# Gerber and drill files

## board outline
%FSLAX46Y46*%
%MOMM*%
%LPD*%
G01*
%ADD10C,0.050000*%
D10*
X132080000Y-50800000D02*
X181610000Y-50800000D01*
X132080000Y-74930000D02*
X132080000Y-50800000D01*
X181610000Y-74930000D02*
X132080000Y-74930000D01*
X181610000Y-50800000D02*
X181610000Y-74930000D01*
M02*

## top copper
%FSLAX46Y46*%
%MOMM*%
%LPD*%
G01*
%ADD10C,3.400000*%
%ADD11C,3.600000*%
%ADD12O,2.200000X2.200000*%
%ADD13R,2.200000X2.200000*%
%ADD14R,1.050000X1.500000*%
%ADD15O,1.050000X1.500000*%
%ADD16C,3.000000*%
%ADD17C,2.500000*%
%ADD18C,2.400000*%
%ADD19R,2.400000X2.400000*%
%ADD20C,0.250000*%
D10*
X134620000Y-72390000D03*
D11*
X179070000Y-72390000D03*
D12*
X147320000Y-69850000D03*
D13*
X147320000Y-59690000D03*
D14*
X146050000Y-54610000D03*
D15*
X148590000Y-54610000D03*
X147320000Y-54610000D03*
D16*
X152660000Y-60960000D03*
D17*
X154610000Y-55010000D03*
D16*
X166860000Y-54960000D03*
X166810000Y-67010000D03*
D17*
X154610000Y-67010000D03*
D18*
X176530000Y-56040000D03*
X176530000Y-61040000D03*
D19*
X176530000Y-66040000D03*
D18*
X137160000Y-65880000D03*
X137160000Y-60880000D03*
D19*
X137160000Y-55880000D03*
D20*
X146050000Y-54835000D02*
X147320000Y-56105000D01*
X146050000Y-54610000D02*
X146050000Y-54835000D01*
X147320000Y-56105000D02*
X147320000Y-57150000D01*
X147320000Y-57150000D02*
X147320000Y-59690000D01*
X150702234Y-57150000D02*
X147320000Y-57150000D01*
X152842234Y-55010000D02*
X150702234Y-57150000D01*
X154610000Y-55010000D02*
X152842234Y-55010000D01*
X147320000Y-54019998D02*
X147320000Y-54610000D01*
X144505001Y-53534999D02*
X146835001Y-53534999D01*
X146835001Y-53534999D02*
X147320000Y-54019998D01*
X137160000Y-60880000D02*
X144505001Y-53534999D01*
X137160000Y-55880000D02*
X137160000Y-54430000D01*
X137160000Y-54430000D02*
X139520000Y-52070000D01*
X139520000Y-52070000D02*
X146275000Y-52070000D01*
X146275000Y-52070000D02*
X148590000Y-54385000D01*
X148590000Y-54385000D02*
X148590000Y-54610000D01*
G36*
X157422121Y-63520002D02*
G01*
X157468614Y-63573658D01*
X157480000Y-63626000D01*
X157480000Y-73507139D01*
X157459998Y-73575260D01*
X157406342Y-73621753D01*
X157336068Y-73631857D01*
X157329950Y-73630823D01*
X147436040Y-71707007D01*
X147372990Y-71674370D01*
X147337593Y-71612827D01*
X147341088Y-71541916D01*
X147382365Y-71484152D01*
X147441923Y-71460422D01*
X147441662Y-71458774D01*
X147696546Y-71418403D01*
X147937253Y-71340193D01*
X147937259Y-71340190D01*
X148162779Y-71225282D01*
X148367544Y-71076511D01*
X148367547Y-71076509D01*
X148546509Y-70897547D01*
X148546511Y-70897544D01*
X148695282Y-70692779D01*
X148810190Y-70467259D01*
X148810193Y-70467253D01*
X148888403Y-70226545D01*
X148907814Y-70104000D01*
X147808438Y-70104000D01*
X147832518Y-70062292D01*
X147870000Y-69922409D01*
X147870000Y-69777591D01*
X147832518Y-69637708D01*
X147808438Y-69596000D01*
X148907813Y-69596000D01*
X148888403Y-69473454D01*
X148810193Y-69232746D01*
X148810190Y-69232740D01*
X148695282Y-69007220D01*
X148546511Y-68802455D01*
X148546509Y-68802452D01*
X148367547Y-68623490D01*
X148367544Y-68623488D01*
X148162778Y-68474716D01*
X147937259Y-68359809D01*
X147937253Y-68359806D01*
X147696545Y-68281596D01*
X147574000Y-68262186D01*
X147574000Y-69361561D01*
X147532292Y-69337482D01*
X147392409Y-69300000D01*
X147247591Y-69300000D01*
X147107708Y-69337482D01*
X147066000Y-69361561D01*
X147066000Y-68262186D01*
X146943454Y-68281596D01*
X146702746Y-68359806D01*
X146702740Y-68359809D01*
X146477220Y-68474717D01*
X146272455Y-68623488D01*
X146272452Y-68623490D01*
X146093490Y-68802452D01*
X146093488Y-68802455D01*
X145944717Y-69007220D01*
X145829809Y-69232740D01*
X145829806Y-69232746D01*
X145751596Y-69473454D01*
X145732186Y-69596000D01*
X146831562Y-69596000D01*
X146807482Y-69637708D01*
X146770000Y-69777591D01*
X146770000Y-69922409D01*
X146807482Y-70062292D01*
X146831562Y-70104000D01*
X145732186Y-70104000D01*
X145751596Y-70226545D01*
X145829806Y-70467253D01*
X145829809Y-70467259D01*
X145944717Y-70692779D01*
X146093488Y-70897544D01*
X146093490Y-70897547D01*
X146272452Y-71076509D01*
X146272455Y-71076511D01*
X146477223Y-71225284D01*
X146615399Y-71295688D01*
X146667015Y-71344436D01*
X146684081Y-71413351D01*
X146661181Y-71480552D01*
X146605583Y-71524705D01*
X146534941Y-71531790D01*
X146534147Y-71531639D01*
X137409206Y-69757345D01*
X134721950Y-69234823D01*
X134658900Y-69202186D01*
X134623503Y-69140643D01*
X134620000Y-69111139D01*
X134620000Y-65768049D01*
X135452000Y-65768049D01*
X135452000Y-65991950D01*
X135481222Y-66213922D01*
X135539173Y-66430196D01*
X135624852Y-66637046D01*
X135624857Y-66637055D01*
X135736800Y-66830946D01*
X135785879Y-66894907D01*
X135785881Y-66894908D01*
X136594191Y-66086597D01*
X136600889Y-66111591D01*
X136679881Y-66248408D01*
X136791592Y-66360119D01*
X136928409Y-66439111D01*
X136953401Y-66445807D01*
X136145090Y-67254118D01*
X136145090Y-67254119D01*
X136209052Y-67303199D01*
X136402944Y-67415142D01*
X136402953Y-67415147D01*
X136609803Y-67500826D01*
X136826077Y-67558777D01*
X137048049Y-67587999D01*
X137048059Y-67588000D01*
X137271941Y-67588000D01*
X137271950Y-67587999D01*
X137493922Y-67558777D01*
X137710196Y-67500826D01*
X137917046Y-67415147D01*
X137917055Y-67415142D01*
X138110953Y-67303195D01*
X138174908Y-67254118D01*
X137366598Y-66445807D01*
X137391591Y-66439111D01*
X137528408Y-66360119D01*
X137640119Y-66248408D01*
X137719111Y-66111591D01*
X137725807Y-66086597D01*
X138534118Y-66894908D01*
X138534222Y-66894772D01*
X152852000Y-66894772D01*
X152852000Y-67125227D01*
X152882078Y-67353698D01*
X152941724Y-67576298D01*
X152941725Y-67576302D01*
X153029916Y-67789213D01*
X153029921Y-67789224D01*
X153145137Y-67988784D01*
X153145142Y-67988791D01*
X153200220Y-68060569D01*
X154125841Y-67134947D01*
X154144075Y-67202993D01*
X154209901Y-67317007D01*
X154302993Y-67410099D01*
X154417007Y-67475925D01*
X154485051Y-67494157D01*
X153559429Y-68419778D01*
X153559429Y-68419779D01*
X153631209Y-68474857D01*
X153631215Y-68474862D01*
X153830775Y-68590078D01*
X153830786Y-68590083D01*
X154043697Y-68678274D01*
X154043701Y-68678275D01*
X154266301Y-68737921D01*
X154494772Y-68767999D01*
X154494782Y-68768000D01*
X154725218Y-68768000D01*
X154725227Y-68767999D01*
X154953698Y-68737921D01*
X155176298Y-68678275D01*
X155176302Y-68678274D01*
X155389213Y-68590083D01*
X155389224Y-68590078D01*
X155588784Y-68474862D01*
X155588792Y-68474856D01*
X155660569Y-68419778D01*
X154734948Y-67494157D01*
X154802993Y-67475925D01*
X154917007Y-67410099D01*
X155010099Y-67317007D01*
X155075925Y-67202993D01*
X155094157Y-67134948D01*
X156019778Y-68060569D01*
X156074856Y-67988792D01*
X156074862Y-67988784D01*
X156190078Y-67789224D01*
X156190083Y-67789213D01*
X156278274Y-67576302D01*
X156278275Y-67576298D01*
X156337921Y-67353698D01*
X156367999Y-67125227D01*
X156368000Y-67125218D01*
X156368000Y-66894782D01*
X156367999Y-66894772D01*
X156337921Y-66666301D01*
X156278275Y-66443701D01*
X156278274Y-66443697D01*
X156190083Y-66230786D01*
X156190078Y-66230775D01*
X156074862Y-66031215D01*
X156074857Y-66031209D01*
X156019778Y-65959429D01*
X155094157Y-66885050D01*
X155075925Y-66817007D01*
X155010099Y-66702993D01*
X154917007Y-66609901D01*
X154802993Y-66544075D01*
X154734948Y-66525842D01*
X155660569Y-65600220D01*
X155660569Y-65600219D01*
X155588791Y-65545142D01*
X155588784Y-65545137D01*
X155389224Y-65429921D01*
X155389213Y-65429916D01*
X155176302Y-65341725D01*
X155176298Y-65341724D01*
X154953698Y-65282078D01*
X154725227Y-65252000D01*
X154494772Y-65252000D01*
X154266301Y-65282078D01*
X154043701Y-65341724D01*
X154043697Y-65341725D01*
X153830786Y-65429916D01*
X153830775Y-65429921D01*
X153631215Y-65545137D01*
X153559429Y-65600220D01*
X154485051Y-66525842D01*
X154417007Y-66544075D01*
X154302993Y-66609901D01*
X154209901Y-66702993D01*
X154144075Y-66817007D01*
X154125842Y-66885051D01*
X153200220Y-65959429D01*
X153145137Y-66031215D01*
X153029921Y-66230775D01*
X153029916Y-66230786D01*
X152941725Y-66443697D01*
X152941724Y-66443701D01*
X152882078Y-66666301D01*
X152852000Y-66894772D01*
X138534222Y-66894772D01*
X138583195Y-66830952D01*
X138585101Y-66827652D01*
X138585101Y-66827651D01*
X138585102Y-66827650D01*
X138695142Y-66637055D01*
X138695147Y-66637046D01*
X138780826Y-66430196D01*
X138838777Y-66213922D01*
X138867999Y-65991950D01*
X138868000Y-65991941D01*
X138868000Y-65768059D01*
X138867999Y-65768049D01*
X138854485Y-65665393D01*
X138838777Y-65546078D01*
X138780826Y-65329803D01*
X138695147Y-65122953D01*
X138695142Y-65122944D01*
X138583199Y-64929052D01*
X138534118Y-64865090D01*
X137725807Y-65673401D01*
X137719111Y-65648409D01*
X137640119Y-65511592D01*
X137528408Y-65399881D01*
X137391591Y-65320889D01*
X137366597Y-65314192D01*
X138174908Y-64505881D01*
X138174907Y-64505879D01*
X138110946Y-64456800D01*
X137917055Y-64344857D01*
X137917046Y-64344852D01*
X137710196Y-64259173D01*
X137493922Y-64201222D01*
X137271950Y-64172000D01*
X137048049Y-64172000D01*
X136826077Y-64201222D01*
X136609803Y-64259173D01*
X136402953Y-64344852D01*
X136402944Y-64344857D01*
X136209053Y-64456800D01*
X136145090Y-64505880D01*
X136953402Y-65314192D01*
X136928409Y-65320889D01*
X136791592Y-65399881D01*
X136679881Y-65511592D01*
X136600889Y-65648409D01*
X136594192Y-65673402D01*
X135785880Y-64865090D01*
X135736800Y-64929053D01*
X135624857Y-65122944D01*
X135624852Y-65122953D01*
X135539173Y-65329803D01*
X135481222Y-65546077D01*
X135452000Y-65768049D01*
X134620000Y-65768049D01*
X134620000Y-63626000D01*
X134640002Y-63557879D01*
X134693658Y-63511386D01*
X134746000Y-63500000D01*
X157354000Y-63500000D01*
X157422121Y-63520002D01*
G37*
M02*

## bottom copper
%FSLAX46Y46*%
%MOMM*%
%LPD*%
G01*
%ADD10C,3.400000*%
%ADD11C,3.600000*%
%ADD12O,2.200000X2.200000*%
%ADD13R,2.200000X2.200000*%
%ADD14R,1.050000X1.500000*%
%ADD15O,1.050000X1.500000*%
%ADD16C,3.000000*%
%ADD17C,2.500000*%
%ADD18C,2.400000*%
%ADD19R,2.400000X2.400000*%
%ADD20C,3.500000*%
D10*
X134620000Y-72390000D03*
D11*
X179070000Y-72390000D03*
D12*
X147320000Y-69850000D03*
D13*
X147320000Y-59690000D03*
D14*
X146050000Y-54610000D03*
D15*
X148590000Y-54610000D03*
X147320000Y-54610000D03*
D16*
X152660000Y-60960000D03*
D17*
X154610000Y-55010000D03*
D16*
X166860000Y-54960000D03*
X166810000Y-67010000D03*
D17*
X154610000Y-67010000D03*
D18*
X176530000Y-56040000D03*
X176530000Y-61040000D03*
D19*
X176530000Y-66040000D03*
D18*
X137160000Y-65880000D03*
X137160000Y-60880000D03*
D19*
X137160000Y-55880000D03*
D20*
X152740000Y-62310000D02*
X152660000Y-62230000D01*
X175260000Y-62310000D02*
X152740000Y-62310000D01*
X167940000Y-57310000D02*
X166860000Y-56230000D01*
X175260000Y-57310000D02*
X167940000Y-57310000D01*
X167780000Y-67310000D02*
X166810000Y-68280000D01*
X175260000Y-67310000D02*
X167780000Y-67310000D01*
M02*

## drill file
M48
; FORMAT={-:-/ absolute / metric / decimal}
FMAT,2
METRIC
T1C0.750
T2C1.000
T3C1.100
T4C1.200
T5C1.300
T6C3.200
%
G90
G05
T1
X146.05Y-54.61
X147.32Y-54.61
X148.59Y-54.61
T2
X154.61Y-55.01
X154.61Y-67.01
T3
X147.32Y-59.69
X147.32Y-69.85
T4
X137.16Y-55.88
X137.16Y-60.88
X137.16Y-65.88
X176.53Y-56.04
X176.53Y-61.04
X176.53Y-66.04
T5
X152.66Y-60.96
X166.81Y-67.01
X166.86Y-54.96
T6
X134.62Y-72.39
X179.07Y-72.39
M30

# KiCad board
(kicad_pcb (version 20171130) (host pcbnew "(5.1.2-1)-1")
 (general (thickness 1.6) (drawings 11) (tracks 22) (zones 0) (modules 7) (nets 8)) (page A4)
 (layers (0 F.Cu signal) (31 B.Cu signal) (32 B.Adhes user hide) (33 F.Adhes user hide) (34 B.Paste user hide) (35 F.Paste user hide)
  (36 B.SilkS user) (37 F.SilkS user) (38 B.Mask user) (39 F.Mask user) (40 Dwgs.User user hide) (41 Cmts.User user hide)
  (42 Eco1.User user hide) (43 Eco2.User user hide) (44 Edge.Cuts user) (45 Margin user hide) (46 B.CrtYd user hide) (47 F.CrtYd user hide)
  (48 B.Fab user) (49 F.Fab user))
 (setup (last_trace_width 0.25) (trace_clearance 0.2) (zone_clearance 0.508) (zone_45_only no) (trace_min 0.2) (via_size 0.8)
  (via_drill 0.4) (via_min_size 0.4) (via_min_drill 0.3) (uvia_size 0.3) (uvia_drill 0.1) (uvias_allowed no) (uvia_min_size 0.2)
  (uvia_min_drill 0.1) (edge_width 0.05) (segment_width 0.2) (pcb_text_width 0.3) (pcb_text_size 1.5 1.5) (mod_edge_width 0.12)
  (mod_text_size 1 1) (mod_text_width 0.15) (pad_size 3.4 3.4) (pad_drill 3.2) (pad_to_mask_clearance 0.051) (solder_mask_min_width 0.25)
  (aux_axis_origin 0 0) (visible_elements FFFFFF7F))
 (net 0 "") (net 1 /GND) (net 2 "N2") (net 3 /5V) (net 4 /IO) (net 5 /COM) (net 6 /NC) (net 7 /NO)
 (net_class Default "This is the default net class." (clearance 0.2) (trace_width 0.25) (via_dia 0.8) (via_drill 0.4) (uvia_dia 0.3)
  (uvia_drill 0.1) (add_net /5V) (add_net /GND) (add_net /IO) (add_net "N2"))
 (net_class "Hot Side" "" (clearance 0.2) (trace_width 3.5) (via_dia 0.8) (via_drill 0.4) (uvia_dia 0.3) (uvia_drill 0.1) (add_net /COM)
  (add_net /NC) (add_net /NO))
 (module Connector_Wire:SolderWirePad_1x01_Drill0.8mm (layer F.Cu) (at 134.62 72.39)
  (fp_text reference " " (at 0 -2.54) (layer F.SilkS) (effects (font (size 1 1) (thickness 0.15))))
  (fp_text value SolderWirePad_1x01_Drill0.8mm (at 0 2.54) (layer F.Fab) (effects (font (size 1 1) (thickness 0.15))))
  (pad 1 thru_hole circle (at 0 0) (size 3.4 3.4) (drill 3.2) (layers *.Cu *.Mask)))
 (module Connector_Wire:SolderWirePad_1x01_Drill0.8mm (layer F.Cu) (at 179.07 72.39)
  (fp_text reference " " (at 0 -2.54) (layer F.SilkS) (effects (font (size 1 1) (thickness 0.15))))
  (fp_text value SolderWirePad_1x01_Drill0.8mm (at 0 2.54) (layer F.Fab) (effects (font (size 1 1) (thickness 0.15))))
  (pad 1 thru_hole circle (at 0 0) (size 3.6 3.6) (drill 3.2) (layers *.Cu *.Mask)))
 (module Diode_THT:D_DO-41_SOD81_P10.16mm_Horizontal (layer F.Cu) (at 147.32 59.69 270)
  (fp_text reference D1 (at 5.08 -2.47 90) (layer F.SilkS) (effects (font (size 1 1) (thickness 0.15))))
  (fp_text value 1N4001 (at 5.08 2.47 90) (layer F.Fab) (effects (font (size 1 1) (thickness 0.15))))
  (pad 2 thru_hole oval (at 10.16 0 270) (size 2.2 2.2) (drill 1.1) (layers *.Cu *.Mask) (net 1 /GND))
  (pad 1 thru_hole rect (at 0 0 270) (size 2.2 2.2) (drill 1.1) (layers *.Cu *.Mask) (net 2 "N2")))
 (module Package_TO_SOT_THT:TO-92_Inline (layer F.Cu) (at 146.05 54.61)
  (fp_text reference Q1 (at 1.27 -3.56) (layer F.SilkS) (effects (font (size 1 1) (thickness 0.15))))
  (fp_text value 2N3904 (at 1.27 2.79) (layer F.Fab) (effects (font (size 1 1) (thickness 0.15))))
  (pad 1 thru_hole rect (at 0 0) (size 1.05 1.5) (drill 0.75) (layers *.Cu *.Mask) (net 2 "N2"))
  (pad 3 thru_hole oval (at 2.54 0) (size 1.05 1.5) (drill 0.75) (layers *.Cu *.Mask) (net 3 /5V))
  (pad 2 thru_hole oval (at 1.27 0) (size 1.05 1.5) (drill 0.75) (layers *.Cu *.Mask) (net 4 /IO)))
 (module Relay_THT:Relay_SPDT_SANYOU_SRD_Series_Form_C (layer F.Cu) (at 152.66 60.96)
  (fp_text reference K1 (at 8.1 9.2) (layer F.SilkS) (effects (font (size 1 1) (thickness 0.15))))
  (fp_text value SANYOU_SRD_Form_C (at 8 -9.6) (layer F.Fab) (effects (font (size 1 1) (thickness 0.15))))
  (pad 1 thru_hole circle (at 0 0 90) (size 3 3) (drill 1.3) (layers *.Cu *.Mask) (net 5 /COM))
  (pad 5 thru_hole circle (at 1.95 -5.95 90) (size 2.5 2.5) (drill 1) (layers *.Cu *.Mask) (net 2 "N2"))
  (pad 4 thru_hole circle (at 14.2 -6 90) (size 3 3) (drill 1.3) (layers *.Cu *.Mask) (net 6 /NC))
  (pad 3 thru_hole circle (at 14.15 6.05 90) (size 3 3) (drill 1.3) (layers *.Cu *.Mask) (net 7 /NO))
  (pad 2 thru_hole circle (at 1.95 6.05 90) (size 2.5 2.5) (drill 1) (layers *.Cu *.Mask) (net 1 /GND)))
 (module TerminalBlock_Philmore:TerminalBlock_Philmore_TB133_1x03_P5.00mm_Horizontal (layer F.Cu) (at 176.53 66.04 90)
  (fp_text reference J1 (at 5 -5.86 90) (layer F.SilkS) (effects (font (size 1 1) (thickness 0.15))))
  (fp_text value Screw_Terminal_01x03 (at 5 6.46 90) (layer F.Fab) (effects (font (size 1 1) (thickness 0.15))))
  (pad 3 thru_hole circle (at 10 0 90) (size 2.4 2.4) (drill 1.2) (layers *.Cu *.Mask) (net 6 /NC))
  (pad 2 thru_hole circle (at 5 0 90) (size 2.4 2.4) (drill 1.2) (layers *.Cu *.Mask) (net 5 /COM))
  (pad 1 thru_hole rect (at 0 0 90) (size 2.4 2.4) (drill 1.2) (layers *.Cu *.Mask) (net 7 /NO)))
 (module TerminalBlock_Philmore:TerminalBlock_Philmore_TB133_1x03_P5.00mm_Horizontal (layer F.Cu) (at 137.16 55.88 270)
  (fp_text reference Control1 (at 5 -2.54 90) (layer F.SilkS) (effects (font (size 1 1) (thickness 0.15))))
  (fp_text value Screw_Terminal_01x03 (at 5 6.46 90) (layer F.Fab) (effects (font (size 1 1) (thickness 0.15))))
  (pad 3 thru_hole circle (at 10 0 270) (size 2.4 2.4) (drill 1.2) (layers *.Cu *.Mask) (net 1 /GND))
  (pad 2 thru_hole circle (at 5 0 270) (size 2.4 2.4) (drill 1.2) (layers *.Cu *.Mask) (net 4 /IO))
  (pad 1 thru_hole rect (at 0 0 270) (size 2.4 2.4) (drill 1.2) (layers *.Cu *.Mask) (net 3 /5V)))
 (gr_line (start 132.08 50.8) (end 181.61 50.8) (layer Edge.Cuts) (width 0.05))
 (gr_line (start 132.08 74.93) (end 132.08 50.8) (layer Edge.Cuts) (width 0.05))
 (gr_line (start 181.61 74.93) (end 132.08 74.93) (layer Edge.Cuts) (width 0.05))
 (gr_line (start 181.61 50.8) (end 181.61 74.93) (layer Edge.Cuts) (width 0.05))
 (segment (start 146.05 54.835) (end 147.32 56.105) (width 0.25) (layer F.Cu) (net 2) (status 10))
 (segment (start 146.05 54.61) (end 146.05 54.835) (width 0.25) (layer F.Cu) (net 2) (status 30))
 (segment (start 147.32 56.105) (end 147.32 57.15) (width 0.25) (layer F.Cu) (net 2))
 (segment (start 147.32 57.15) (end 147.32 59.69) (width 0.25) (layer F.Cu) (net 2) (status 20))
 (segment (start 150.702234 57.15) (end 147.32 57.15) (width 0.25) (layer F.Cu) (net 2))
 (segment (start 152.842234 55.01) (end 150.702234 57.15) (width 0.25) (layer F.Cu) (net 2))
 (segment (start 154.61 55.01) (end 152.842234 55.01) (width 0.25) (layer F.Cu) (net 2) (status 10))
 (segment (start 147.32 54.019998) (end 147.32 54.61) (width 0.25) (layer F.Cu) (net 4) (status 30))
 (segment (start 144.505001 53.534999) (end 146.835001 53.534999) (width 0.25) (layer F.Cu) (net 4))
 (segment (start 146.835001 53.534999) (end 147.32 54.019998) (width 0.25) (layer F.Cu) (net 4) (status 20))
 (segment (start 137.16 60.88) (end 144.505001 53.534999) (width 0.25) (layer F.Cu) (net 4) (status 10))
 (segment (start 137.16 55.88) (end 137.16 54.43) (width 0.25) (layer F.Cu) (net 3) (status 10))
 (segment (start 137.16 54.43) (end 139.52 52.07) (width 0.25) (layer F.Cu) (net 3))
 (segment (start 139.52 52.07) (end 146.275 52.07) (width 0.25) (layer F.Cu) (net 3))
 (segment (start 146.275 52.07) (end 148.59 54.385) (width 0.25) (layer F.Cu) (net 3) (status 20))
 (segment (start 148.59 54.385) (end 148.59 54.61) (width 0.25) (layer F.Cu) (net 3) (status 30))
 (segment (start 152.74 62.31) (end 152.66 62.23) (width 3.5) (layer B.Cu) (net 5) (status 30))
 (segment (start 175.26 62.31) (end 152.74 62.31) (width 3.5) (layer B.Cu) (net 5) (status 20))
 (segment (start 167.94 57.31) (end 166.86 56.23) (width 3.5) (layer B.Cu) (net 6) (status 20))
 (segment (start 175.26 57.31) (end 167.94 57.31) (width 3.5) (layer B.Cu) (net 6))
 (segment (start 167.78 67.31) (end 166.81 68.28) (width 3.5) (layer B.Cu) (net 7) (status 30))
 (segment (start 175.26 67.31) (end 167.78 67.31) (width 3.5) (layer B.Cu) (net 7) (status 20))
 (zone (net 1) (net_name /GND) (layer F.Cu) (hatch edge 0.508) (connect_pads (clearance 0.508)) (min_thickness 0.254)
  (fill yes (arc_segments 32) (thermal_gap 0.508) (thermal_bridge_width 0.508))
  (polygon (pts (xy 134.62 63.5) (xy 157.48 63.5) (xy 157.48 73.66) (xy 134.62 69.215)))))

